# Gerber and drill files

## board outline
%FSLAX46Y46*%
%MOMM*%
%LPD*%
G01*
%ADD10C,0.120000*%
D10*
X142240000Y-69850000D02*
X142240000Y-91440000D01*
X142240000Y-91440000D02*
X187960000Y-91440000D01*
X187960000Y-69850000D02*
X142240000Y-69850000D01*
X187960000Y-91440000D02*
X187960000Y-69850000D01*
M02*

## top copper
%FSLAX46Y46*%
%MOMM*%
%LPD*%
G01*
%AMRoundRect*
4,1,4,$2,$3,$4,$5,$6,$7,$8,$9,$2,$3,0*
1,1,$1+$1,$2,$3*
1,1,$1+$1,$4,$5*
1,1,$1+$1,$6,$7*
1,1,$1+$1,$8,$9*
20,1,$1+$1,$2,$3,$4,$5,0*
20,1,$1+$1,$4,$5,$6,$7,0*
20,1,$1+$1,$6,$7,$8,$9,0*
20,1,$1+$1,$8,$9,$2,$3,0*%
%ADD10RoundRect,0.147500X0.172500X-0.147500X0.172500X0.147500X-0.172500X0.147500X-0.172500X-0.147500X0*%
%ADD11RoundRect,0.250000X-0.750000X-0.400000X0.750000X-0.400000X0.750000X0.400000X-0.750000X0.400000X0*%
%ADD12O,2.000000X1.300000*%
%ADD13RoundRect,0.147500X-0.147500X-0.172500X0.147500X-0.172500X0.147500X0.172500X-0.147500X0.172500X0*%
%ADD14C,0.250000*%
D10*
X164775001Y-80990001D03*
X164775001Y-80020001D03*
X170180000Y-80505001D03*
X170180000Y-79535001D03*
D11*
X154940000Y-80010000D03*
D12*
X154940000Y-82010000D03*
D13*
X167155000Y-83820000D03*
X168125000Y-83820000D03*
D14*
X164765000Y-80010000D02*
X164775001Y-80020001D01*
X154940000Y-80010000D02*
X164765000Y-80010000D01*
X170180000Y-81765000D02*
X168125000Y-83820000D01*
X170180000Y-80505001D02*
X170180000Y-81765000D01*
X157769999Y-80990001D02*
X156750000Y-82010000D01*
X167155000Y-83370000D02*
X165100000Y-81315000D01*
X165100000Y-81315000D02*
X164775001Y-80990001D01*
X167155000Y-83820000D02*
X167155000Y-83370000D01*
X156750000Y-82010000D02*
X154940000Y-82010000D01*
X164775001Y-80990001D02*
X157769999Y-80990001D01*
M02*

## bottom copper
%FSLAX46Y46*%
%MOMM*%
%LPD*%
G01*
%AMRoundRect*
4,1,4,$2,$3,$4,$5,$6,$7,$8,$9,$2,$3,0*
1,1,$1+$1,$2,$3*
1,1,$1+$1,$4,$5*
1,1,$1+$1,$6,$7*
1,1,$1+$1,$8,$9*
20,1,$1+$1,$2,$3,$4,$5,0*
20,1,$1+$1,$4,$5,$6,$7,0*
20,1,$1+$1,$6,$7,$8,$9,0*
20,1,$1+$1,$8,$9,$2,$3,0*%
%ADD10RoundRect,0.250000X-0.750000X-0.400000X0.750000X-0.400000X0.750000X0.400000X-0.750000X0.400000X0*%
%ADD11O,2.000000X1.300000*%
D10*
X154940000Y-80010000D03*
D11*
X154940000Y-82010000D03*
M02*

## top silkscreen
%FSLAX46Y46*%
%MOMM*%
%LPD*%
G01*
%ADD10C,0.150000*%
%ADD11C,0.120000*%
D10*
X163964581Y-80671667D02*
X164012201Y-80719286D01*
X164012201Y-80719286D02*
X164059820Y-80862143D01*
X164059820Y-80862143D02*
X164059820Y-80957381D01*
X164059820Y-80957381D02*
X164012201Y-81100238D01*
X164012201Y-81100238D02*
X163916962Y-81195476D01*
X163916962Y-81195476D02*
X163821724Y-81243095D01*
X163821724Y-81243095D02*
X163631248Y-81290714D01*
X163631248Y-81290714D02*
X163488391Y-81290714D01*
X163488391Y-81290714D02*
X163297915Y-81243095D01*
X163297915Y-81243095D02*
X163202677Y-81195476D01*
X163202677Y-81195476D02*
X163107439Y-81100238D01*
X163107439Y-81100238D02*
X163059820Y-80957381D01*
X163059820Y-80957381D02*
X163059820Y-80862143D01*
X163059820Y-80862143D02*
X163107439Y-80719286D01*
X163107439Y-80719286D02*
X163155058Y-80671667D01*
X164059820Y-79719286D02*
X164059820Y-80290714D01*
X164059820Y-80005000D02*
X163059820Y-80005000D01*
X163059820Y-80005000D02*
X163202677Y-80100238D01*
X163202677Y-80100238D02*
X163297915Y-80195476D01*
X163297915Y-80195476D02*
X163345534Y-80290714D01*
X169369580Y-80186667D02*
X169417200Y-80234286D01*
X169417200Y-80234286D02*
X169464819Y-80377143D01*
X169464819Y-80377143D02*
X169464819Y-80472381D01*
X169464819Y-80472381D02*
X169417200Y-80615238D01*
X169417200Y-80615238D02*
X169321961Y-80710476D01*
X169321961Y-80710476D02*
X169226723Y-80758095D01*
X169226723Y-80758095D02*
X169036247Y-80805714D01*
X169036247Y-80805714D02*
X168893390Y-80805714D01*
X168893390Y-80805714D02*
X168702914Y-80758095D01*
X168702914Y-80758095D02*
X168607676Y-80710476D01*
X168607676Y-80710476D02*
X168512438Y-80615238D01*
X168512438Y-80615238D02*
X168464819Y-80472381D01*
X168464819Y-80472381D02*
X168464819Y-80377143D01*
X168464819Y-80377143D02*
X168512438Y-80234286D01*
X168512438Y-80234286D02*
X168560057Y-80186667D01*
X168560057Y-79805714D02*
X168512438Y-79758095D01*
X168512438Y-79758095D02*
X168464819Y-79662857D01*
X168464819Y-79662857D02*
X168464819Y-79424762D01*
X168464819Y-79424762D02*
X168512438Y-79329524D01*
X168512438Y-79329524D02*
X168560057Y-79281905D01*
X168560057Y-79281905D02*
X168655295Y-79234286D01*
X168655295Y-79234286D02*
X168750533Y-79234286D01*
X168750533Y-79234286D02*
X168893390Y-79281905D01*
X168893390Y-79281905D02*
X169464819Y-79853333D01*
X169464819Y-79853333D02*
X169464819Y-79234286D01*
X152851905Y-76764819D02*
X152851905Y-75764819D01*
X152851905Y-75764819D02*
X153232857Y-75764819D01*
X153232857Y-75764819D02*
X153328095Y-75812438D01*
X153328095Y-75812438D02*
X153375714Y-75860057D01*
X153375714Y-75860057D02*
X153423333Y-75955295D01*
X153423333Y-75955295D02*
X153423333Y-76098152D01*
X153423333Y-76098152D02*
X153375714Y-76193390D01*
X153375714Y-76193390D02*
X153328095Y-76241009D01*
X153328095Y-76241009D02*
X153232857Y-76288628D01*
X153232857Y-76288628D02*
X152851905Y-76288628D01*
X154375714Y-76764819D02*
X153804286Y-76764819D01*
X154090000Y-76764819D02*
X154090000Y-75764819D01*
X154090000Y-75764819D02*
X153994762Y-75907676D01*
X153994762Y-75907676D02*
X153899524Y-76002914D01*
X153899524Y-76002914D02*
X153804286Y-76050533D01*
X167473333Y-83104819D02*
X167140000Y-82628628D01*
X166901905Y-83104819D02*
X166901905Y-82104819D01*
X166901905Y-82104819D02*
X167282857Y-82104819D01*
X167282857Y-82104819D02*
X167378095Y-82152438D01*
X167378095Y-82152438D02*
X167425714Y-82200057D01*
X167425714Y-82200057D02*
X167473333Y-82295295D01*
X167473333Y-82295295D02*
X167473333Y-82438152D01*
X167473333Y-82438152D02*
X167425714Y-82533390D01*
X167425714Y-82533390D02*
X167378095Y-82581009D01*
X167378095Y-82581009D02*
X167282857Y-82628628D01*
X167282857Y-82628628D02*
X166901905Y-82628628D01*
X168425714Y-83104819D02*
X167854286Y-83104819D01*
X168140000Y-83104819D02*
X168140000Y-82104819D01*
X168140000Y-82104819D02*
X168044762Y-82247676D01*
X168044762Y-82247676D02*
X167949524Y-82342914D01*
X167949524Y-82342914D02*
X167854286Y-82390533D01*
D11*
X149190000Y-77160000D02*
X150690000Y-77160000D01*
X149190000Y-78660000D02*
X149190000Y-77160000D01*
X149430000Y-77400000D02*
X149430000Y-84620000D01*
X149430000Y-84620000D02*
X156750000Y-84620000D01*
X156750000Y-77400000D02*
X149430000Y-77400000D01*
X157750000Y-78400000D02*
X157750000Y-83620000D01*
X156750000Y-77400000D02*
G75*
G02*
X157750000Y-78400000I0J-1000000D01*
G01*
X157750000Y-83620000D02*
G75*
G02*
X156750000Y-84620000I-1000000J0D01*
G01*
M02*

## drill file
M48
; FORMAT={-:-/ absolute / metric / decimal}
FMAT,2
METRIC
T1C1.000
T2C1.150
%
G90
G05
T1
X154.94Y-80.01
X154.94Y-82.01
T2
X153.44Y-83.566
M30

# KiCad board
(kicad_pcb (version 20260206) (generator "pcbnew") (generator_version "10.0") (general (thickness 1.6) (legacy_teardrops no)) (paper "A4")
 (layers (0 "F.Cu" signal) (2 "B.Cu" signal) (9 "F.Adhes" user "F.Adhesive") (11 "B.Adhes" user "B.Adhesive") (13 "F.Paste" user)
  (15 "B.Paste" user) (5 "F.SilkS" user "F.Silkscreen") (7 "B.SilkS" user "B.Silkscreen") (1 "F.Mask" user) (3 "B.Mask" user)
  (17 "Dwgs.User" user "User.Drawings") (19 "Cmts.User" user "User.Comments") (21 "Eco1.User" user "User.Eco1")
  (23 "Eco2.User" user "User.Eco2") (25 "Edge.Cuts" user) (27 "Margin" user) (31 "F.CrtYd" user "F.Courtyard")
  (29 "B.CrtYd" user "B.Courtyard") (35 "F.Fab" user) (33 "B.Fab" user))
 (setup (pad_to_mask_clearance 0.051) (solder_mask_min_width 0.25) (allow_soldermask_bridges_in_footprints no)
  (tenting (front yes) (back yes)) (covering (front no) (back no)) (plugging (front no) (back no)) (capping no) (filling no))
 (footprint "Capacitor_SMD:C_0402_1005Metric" (layer "F.Cu") (at 164.775001 80.505001 90)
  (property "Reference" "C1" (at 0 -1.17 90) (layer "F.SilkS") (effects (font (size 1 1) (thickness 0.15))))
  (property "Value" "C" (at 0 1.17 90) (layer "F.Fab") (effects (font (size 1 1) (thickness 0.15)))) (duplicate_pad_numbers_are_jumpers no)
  (pad "1" smd roundrect (at -0.485 0 90) (size 0.59 0.64) (layers "F.Cu" "F.Mask" "F.Paste") (roundrect_rratio 0.25) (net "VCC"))
  (pad "2" smd roundrect (at 0.485 0 90) (size 0.59 0.64) (layers "F.Cu" "F.Mask" "F.Paste") (roundrect_rratio 0.25) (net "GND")))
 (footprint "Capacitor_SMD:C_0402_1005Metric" (layer "F.Cu") (at 170.18 80.020001 90)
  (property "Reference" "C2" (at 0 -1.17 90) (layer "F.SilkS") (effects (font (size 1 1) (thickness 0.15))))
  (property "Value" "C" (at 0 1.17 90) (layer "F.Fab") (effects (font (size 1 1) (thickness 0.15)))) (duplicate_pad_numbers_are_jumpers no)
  (pad "1" smd roundrect (at -0.485 0 90) (size 0.59 0.64) (layers "F.Cu" "F.Mask" "F.Paste") (roundrect_rratio 0.25) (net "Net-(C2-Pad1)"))
  (pad "2" smd roundrect (at 0.485 0 90) (size 0.59 0.64) (layers "F.Cu" "F.Mask" "F.Paste") (roundrect_rratio 0.25) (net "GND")))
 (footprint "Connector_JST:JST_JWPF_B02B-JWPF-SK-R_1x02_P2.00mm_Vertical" (layer "F.Cu") (at 154.94 80.01)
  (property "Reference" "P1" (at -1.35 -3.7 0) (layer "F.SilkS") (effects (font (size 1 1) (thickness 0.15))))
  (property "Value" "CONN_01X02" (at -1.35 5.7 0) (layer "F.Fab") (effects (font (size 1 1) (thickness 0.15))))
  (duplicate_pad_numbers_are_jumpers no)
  (fp_line (start -5.75 -2.85) (end -4.25 -2.85) (stroke (width 0.12) (type solid)) (layer "F.SilkS"))
  (fp_line (start -5.75 -1.35) (end -5.75 -2.85) (stroke (width 0.12) (type solid)) (layer "F.SilkS"))
  (fp_line (start -5.51 -2.61) (end -5.51 4.61) (stroke (width 0.12) (type solid)) (layer "F.SilkS"))
  (fp_line (start -5.51 4.61) (end 1.81 4.61) (stroke (width 0.12) (type solid)) (layer "F.SilkS"))
  (fp_line (start 1.81 -2.61) (end -5.51 -2.61) (stroke (width 0.12) (type solid)) (layer "F.SilkS"))
  (fp_line (start 2.81 -1.61) (end 2.81 3.61) (stroke (width 0.12) (type solid)) (layer "F.SilkS"))
  (fp_arc (start 1.81 -2.61) (mid 2.517107 -2.317107) (end 2.81 -1.61) (stroke (width 0.12) (type solid)) (layer "F.SilkS"))
  (fp_arc (start 2.81 3.61) (mid 2.517107 4.317107) (end 1.81 4.61) (stroke (width 0.12) (type solid)) (layer "F.SilkS"))
  (pad "" np_thru_hole circle (at -1.5 3.556) (size 1.15 1.15) (drill 1.15) (layers "*.Cu" "*.Mask"))
  (pad "1" thru_hole roundrect (at 0 0) (size 2 1.3) (drill 1) (layers "*.Cu" "*.Mask") (remove_unused_layers no)
   (roundrect_rratio 0.192308) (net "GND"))
  (pad "2" thru_hole oval (at 0 2) (size 2 1.3) (drill 1) (layers "*.Cu" "*.Mask") (remove_unused_layers no) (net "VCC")))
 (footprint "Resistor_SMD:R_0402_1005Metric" (layer "F.Cu") (at 167.64 83.82)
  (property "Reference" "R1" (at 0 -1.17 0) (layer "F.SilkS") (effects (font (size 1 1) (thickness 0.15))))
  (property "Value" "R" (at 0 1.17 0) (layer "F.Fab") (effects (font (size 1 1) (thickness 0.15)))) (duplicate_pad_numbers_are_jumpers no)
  (pad "1" smd roundrect (at -0.485 0) (size 0.59 0.64) (layers "F.Cu" "F.Mask" "F.Paste") (roundrect_rratio 0.25) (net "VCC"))
  (pad "2" smd roundrect (at 0.485 0) (size 0.59 0.64) (layers "F.Cu" "F.Mask" "F.Paste") (roundrect_rratio 0.25) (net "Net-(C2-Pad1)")))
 (gr_line (start 142.24 69.85) (end 142.24 91.44) (stroke (width 0.12) (type solid)) (layer "Edge.Cuts"))
 (gr_line (start 142.24 91.44) (end 187.96 91.44) (stroke (width 0.12) (type solid)) (layer "Edge.Cuts"))
 (gr_line (start 187.96 69.85) (end 142.24 69.85) (stroke (width 0.12) (type solid)) (layer "Edge.Cuts"))
 (gr_line (start 187.96 91.44) (end 187.96 69.85) (stroke (width 0.12) (type solid)) (layer "Edge.Cuts"))
 (segment (start 164.765 80.01) (end 164.775001 80.020001) (width 0.25) (layer "F.Cu") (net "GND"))
 (segment (start 154.94 80.01) (end 164.765 80.01) (width 0.25) (layer "F.Cu") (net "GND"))
 (segment (start 170.18 81.765) (end 168.125 83.82) (width 0.25) (layer "F.Cu") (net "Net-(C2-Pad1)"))
 (segment (start 170.18 80.505001) (end 170.18 81.765) (width 0.25) (layer "F.Cu") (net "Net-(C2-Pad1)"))
 (segment (start 157.769999 80.990001) (end 156.75 82.01) (width 0.25) (layer "F.Cu") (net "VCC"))
 (segment (start 167.155 83.37) (end 165.1 81.315) (width 0.25) (layer "F.Cu") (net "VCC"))
 (segment (start 165.1 81.315) (end 164.775001 80.990001) (width 0.25) (layer "F.Cu") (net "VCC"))
 (segment (start 167.155 83.82) (end 167.155 83.37) (width 0.25) (layer "F.Cu") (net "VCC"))
 (segment (start 156.75 82.01) (end 154.94 82.01) (width 0.25) (layer "F.Cu") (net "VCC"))
 (segment (start 164.775001 80.990001) (end 157.769999 80.990001) (width 0.25) (layer "F.Cu") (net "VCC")))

